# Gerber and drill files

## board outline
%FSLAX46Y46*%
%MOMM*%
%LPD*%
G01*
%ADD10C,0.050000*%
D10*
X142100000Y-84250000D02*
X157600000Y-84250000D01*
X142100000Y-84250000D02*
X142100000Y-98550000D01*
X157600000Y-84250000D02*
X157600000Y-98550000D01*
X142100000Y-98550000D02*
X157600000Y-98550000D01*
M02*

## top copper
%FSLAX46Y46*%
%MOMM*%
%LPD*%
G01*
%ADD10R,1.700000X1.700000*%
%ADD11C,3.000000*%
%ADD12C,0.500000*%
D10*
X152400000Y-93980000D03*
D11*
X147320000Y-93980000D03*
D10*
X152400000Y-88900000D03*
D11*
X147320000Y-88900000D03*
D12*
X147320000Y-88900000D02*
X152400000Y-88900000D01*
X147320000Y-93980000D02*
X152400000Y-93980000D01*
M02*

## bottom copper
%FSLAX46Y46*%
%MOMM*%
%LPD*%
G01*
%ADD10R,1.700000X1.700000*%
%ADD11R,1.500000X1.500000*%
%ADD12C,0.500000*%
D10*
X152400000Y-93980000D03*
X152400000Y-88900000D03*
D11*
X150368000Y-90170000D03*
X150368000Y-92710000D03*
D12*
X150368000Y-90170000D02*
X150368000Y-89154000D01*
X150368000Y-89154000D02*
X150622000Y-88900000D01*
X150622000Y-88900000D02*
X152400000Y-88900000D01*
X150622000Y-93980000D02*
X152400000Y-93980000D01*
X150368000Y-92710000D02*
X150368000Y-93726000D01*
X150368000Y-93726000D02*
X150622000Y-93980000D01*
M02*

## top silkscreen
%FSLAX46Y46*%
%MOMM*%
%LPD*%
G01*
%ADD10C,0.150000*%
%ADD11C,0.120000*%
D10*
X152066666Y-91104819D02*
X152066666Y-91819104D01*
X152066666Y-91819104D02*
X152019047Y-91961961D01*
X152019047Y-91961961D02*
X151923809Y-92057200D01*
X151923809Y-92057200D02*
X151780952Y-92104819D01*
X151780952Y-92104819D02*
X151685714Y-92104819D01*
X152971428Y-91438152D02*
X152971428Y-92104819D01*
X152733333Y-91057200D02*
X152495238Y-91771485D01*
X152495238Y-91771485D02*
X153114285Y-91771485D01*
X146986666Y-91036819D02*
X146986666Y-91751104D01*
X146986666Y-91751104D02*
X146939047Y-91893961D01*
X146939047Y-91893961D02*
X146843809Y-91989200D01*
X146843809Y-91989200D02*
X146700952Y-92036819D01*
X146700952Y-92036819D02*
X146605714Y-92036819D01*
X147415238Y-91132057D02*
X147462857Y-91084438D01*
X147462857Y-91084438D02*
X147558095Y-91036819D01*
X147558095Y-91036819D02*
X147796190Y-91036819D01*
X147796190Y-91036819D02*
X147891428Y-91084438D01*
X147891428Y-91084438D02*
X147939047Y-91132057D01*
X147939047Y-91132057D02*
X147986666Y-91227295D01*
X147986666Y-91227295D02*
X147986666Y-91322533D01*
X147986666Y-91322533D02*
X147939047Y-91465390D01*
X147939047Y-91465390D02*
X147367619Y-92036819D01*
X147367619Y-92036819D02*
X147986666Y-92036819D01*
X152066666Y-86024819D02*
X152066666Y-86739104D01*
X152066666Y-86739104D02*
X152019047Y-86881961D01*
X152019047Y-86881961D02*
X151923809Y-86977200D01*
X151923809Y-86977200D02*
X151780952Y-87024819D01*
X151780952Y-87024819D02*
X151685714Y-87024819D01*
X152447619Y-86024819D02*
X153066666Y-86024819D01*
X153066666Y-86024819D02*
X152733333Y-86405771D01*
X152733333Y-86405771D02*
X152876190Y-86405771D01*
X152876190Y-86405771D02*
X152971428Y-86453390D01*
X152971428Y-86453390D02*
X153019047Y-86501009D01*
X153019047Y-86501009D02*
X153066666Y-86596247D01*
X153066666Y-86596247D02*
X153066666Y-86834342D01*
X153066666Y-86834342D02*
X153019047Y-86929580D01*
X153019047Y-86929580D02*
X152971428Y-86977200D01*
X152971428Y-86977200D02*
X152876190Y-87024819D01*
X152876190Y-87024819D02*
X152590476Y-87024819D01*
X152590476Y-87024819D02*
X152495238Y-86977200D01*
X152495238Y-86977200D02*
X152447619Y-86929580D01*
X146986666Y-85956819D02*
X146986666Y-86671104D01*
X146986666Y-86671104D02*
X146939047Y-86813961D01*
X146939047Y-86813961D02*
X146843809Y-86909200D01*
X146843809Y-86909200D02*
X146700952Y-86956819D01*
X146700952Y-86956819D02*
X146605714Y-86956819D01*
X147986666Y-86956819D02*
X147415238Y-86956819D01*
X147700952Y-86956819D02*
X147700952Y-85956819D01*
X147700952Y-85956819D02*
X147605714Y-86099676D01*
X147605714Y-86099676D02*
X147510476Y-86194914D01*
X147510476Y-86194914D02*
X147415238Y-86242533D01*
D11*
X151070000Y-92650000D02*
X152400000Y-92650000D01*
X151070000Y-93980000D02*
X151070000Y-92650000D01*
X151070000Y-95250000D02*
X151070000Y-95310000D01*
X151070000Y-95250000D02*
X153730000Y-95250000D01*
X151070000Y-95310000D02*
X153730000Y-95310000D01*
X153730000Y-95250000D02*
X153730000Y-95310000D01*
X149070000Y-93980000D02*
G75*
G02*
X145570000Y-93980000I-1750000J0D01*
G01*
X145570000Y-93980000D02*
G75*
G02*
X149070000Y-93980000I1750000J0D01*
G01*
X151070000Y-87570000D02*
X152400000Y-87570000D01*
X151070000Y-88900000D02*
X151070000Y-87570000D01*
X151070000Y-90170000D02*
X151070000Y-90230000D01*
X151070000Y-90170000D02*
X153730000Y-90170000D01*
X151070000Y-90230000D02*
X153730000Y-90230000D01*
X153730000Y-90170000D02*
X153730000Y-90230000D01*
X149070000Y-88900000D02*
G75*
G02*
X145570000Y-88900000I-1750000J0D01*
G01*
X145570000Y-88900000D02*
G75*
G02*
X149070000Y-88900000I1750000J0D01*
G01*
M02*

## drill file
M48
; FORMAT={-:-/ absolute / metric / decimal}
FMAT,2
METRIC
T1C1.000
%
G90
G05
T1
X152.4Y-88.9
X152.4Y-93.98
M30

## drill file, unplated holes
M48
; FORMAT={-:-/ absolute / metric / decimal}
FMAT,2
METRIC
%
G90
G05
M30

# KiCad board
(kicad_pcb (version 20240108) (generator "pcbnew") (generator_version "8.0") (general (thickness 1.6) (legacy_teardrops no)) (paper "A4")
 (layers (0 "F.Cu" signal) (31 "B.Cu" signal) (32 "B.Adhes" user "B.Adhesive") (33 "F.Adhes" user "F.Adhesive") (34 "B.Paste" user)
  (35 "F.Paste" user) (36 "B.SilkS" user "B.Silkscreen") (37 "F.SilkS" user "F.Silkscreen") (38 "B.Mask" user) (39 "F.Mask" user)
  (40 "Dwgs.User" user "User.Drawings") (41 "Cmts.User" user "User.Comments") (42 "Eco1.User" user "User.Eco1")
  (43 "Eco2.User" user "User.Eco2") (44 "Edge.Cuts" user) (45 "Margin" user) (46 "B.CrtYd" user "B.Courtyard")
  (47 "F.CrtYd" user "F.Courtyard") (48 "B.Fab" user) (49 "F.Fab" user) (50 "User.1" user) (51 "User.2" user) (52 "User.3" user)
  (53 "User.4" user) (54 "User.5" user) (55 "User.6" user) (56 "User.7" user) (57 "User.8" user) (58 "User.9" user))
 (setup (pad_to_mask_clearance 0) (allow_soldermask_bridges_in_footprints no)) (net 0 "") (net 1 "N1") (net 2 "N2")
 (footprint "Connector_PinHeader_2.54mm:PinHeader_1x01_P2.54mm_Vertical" (layer "F.Cu") (at 152.4 93.98)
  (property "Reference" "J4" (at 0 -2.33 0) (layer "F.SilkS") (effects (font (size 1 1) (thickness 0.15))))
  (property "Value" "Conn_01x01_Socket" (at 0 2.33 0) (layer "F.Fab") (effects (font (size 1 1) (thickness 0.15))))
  (fp_line (start -1.33 -1.33) (end 0 -1.33) (stroke (width 0.12) (type solid)) (layer "F.SilkS"))
  (fp_line (start -1.33 0) (end -1.33 -1.33) (stroke (width 0.12) (type solid)) (layer "F.SilkS"))
  (fp_line (start -1.33 1.27) (end -1.33 1.33) (stroke (width 0.12) (type solid)) (layer "F.SilkS"))
  (fp_line (start -1.33 1.27) (end 1.33 1.27) (stroke (width 0.12) (type solid)) (layer "F.SilkS"))
  (fp_line (start -1.33 1.33) (end 1.33 1.33) (stroke (width 0.12) (type solid)) (layer "F.SilkS"))
  (fp_line (start 1.33 1.27) (end 1.33 1.33) (stroke (width 0.12) (type solid)) (layer "F.SilkS"))
  (pad "1" thru_hole rect (at 0 0) (size 1.7 1.7) (drill 1) (layers "*.Cu" "*.Mask") (remove_unused_layers no) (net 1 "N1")))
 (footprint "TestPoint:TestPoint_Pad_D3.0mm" (layer "F.Cu") (at 147.32 93.98)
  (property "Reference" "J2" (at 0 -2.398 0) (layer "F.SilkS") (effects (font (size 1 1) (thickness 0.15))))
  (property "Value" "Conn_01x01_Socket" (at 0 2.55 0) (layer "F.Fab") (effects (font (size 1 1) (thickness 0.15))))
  (fp_circle (center 0 0) (end 0 1.75) (stroke (width 0.12) (type solid)) (fill none) (layer "F.SilkS"))
  (pad "1" smd circle (at 0 0) (size 3 3) (layers "F.Cu" "F.Mask") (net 1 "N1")))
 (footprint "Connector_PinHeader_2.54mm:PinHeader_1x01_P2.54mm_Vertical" (layer "F.Cu") (at 152.4 88.9)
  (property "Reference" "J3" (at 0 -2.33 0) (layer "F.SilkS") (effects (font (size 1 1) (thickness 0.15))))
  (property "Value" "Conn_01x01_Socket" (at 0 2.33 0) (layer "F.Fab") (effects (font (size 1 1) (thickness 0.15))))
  (fp_line (start -1.33 -1.33) (end 0 -1.33) (stroke (width 0.12) (type solid)) (layer "F.SilkS"))
  (fp_line (start -1.33 0) (end -1.33 -1.33) (stroke (width 0.12) (type solid)) (layer "F.SilkS"))
  (fp_line (start -1.33 1.27) (end -1.33 1.33) (stroke (width 0.12) (type solid)) (layer "F.SilkS"))
  (fp_line (start -1.33 1.27) (end 1.33 1.27) (stroke (width 0.12) (type solid)) (layer "F.SilkS"))
  (fp_line (start -1.33 1.33) (end 1.33 1.33) (stroke (width 0.12) (type solid)) (layer "F.SilkS"))
  (fp_line (start 1.33 1.27) (end 1.33 1.33) (stroke (width 0.12) (type solid)) (layer "F.SilkS"))
  (pad "1" thru_hole rect (at 0 0) (size 1.7 1.7) (drill 1) (layers "*.Cu" "*.Mask") (remove_unused_layers no) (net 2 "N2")))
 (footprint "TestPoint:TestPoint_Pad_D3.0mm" (layer "F.Cu") (at 147.32 88.9)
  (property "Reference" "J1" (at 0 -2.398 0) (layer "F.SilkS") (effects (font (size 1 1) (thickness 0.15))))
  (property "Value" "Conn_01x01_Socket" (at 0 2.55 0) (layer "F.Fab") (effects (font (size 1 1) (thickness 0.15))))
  (fp_circle (center 0 0) (end 0 1.75) (stroke (width 0.12) (type solid)) (fill none) (layer "F.SilkS"))
  (pad "1" smd circle (at 0 0) (size 3 3) (layers "F.Cu" "F.Mask") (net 2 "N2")))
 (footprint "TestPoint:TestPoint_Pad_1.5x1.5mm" (layer "B.Cu") (at 150.368 90.17 180)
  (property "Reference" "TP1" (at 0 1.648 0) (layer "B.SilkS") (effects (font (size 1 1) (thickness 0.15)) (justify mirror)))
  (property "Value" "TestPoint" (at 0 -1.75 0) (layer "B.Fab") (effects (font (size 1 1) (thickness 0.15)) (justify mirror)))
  (pad "1" smd rect (at 0 0 180) (size 1.5 1.5) (layers "B.Cu" "B.Mask") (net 2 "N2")))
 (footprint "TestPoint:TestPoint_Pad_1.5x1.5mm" (layer "B.Cu") (at 150.368 92.71 180)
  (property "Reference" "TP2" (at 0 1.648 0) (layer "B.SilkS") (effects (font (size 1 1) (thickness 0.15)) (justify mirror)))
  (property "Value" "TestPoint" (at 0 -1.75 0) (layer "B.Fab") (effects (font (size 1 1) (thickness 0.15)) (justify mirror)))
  (pad "1" smd rect (at 0 0 180) (size 1.5 1.5) (layers "B.Cu" "B.Mask") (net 1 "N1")))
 (gr_line (start 142.1 84.25) (end 157.6 84.25) (stroke (width 0.05) (type default)) (layer "Edge.Cuts"))
 (gr_line (start 142.1 84.25) (end 142.1 98.55) (stroke (width 0.05) (type default)) (layer "Edge.Cuts"))
 (gr_line (start 157.6 84.25) (end 157.6 98.55) (stroke (width 0.05) (type default)) (layer "Edge.Cuts"))
 (gr_line (start 142.1 98.55) (end 157.6 98.55) (stroke (width 0.05) (type default)) (layer "Edge.Cuts"))
 (segment (start 147.32 88.9) (end 152.4 88.9) (width 0.5) (layer "F.Cu") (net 2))
 (segment (start 150.368 90.17) (end 150.368 89.154) (width 0.5) (layer "B.Cu") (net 2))
 (segment (start 150.368 89.154) (end 150.622 88.9) (width 0.5) (layer "B.Cu") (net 2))
 (segment (start 150.622 88.9) (end 152.4 88.9) (width 0.5) (layer "B.Cu") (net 2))
 (segment (start 147.32 93.98) (end 152.4 93.98) (width 0.5) (layer "F.Cu") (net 1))
 (segment (start 150.622 93.98) (end 152.4 93.98) (width 0.5) (layer "B.Cu") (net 1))
 (segment (start 150.368 92.71) (end 150.368 93.726) (width 0.5) (layer "B.Cu") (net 1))
 (segment (start 150.368 93.726) (end 150.622 93.98) (width 0.5) (layer "B.Cu") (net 1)))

